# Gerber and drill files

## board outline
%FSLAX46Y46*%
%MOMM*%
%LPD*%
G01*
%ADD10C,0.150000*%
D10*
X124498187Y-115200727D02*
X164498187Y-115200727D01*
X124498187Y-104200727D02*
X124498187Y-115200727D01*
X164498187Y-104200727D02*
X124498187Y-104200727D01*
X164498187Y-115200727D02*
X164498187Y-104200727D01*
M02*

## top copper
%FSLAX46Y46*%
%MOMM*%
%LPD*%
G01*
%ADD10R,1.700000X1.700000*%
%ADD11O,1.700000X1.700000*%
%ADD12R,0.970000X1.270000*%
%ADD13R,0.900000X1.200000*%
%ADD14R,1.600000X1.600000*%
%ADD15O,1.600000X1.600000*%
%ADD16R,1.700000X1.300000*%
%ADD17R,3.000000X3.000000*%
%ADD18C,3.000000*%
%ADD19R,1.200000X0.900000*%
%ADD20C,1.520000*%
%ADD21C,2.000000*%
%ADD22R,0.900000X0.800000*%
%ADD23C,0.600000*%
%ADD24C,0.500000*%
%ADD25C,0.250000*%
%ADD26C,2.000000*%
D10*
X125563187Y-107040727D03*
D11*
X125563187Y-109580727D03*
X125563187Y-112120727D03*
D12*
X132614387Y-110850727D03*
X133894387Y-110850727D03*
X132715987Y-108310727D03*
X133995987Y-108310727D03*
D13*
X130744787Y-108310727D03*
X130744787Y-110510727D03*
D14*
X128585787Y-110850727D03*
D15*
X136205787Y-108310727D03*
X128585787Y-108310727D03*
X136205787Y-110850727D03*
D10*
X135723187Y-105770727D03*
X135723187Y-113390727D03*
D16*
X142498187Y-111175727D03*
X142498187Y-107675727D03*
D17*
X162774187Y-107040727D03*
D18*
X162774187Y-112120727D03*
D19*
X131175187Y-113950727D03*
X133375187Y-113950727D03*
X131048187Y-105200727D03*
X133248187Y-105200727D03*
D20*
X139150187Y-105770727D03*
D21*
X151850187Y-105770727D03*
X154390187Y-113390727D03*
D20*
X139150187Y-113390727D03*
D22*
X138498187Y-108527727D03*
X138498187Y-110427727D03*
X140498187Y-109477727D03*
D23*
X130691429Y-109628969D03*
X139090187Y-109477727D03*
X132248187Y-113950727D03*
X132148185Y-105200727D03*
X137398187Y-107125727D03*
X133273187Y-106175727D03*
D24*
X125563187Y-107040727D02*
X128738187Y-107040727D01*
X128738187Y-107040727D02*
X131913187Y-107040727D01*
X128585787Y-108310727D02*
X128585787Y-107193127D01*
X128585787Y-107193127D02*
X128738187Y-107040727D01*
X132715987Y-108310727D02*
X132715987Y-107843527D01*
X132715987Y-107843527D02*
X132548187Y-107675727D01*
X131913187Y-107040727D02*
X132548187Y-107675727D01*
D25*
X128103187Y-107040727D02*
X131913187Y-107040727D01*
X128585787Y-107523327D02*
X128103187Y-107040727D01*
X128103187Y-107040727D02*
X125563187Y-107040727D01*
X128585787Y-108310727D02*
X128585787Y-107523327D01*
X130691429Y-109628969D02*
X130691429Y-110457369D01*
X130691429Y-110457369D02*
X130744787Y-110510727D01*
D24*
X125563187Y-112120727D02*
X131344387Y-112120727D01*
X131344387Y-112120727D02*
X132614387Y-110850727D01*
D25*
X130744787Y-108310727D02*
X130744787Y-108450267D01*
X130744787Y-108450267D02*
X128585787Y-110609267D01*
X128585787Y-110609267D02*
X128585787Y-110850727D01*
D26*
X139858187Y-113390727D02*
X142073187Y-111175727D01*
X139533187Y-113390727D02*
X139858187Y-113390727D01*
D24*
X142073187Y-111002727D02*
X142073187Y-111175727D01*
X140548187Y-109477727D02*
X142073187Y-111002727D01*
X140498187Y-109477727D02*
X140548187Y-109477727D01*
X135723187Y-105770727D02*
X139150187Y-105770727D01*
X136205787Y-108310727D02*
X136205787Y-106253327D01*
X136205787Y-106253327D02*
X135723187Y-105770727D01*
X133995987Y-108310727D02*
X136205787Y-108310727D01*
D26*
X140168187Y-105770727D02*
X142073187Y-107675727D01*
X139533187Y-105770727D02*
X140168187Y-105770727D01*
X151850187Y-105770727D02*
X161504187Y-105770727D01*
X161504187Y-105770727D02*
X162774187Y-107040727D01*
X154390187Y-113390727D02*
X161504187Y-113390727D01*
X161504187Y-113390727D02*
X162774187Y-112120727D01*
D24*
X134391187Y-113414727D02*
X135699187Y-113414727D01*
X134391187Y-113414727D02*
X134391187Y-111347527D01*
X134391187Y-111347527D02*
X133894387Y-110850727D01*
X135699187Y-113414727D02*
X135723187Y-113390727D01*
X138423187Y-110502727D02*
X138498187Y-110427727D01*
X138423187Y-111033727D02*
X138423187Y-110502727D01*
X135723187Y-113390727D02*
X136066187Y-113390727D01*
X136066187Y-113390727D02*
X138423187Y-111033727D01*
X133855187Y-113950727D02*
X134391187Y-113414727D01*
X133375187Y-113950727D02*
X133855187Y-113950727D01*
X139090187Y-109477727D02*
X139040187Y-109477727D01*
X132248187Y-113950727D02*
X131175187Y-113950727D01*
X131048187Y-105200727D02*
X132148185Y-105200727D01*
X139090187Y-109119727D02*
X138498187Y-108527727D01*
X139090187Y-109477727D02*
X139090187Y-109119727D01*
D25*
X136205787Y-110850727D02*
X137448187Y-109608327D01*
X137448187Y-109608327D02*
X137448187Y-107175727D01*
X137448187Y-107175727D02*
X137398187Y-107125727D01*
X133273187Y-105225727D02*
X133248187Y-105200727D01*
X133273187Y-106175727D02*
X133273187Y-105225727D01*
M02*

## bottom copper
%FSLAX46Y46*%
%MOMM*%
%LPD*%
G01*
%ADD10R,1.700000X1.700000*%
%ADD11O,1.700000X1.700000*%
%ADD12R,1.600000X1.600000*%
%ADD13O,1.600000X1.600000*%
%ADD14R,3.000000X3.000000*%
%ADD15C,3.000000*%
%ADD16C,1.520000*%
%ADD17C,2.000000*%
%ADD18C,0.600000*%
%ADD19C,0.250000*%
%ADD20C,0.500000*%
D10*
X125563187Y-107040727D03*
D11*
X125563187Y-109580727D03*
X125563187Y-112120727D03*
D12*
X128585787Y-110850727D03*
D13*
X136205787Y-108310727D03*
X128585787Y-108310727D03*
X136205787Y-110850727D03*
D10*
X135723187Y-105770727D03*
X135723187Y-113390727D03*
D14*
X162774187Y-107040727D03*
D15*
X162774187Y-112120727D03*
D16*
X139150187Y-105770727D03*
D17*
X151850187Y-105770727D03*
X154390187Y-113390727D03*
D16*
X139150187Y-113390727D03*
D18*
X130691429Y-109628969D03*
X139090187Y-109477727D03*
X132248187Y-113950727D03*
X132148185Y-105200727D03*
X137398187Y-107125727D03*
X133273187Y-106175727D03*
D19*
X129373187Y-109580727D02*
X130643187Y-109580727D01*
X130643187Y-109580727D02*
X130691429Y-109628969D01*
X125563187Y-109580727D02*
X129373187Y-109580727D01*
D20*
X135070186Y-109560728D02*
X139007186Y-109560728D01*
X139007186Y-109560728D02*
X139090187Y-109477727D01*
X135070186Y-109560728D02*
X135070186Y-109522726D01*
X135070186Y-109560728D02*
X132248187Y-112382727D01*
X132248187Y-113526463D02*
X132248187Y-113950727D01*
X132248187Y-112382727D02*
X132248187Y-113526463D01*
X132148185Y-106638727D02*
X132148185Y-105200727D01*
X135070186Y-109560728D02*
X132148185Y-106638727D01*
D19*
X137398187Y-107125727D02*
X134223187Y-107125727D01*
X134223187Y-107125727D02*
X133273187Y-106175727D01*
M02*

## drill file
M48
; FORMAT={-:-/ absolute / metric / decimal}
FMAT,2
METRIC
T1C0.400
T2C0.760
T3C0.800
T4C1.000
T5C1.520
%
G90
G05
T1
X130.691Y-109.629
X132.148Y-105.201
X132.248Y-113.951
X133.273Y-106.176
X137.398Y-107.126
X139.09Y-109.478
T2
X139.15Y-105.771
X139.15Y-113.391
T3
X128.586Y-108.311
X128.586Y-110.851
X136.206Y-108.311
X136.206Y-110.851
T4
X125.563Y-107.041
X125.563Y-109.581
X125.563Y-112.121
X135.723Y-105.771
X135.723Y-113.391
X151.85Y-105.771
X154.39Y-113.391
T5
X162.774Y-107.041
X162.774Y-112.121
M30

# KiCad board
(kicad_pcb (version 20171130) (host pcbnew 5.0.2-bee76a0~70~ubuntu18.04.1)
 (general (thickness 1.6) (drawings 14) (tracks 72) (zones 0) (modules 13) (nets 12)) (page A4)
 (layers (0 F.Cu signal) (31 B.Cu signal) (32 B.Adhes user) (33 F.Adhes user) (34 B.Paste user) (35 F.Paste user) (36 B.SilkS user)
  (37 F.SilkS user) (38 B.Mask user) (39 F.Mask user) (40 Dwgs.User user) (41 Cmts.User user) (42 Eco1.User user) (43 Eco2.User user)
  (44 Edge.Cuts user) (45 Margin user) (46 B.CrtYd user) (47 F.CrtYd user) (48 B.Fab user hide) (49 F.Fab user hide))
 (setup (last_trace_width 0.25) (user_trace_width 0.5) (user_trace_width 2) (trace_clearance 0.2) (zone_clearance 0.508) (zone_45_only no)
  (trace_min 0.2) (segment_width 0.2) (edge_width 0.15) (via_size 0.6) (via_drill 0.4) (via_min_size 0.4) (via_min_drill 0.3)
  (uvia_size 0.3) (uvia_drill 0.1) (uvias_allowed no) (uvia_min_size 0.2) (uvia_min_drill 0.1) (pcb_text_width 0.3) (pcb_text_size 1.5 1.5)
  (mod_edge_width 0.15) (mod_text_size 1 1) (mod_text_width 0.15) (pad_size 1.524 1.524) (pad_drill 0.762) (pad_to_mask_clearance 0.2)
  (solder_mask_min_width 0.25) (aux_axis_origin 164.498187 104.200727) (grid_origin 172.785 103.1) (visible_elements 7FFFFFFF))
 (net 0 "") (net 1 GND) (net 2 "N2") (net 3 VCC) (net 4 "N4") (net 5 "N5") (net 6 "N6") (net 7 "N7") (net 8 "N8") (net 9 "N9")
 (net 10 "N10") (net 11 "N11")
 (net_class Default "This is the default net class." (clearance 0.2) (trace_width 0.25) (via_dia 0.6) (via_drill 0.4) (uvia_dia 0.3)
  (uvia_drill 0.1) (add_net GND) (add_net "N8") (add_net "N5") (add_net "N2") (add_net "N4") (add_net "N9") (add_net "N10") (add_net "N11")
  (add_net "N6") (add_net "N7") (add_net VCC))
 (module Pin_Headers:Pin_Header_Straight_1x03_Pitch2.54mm (layer B.Cu) (at 125.563187 107.040727 180)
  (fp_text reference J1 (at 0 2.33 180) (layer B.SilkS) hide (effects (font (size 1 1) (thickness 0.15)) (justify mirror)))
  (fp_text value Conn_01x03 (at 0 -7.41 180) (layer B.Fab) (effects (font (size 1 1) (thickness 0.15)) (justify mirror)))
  (pad 1 thru_hole rect (at 0 0 180) (size 1.7 1.7) (drill 1) (layers *.Cu *.Mask) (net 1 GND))
  (pad 2 thru_hole oval (at 0 -2.54 180) (size 1.7 1.7) (drill 1) (layers *.Cu *.Mask) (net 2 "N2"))
  (pad 3 thru_hole oval (at 0 -5.08 180) (size 1.7 1.7) (drill 1) (layers *.Cu *.Mask) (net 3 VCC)))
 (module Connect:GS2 (layer F.Cu) (at 133.254387 110.850727 90)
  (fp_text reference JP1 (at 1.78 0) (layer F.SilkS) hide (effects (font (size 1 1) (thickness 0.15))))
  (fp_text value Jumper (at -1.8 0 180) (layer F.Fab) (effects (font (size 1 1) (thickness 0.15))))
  (pad 1 smd rect (at 0 -0.64 90) (size 1.27 0.97) (layers F.Cu F.Paste F.Mask) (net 3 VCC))
  (pad 2 smd rect (at 0 0.64 90) (size 1.27 0.97) (layers F.Cu F.Paste F.Mask) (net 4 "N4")))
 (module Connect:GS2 (layer F.Cu) (at 133.355987 108.310727 90)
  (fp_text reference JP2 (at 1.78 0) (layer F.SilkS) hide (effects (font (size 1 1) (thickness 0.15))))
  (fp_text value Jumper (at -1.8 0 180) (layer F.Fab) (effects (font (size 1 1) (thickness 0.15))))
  (pad 1 smd rect (at 0 -0.64 90) (size 1.27 0.97) (layers F.Cu F.Paste F.Mask) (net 1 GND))
  (pad 2 smd rect (at 0 0.64 90) (size 1.27 0.97) (layers F.Cu F.Paste F.Mask) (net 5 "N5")))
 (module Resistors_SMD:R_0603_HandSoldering (layer F.Cu) (at 130.744787 109.410727 270)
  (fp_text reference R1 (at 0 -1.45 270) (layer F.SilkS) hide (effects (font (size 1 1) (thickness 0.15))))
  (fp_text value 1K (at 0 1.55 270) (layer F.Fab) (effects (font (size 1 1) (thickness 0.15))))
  (pad 1 smd rect (at -1.1 0 270) (size 1.2 0.9) (layers F.Cu F.Paste F.Mask) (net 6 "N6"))
  (pad 2 smd rect (at 1.1 0 270) (size 1.2 0.9) (layers F.Cu F.Paste F.Mask) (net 2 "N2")))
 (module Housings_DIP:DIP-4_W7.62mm (layer B.Cu) (at 128.585787 110.850727)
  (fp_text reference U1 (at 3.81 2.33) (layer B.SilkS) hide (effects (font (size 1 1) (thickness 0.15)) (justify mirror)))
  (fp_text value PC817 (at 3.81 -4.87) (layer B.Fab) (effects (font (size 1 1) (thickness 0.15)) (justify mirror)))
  (pad 1 thru_hole rect (at 0 0) (size 1.6 1.6) (drill 0.8) (layers *.Cu *.Mask) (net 6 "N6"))
  (pad 3 thru_hole oval (at 7.62 -2.54) (size 1.6 1.6) (drill 0.8) (layers *.Cu *.Mask) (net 5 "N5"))
  (pad 2 thru_hole oval (at 0 -2.54) (size 1.6 1.6) (drill 0.8) (layers *.Cu *.Mask) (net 1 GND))
  (pad 4 thru_hole oval (at 7.62 0) (size 1.6 1.6) (drill 0.8) (layers *.Cu *.Mask) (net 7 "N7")))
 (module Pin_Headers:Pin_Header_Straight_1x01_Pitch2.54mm (layer B.Cu) (at 135.723187 105.770727 270)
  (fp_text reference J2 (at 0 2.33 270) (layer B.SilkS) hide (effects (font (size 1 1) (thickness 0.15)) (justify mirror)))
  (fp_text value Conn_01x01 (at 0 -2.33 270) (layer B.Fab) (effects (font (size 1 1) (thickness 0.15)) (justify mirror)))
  (pad 1 thru_hole rect (at 0 0 270) (size 1.7 1.7) (drill 1) (layers *.Cu *.Mask) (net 5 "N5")))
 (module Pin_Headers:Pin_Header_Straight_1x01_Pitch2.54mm (layer B.Cu) (at 135.723187 113.390727)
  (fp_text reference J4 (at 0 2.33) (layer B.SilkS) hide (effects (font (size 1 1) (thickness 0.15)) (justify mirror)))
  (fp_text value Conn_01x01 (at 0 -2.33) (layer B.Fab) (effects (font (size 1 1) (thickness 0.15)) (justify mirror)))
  (pad 1 thru_hole rect (at 0 0) (size 1.7 1.7) (drill 1) (layers *.Cu *.Mask) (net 4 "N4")))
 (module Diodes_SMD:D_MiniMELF (layer F.Cu) (at 142.498187 109.425727 90)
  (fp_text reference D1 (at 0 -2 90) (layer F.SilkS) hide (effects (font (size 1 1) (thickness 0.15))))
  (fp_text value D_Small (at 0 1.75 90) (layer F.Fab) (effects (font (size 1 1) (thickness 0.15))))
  (pad 1 smd rect (at -1.75 0 90) (size 1.3 1.7) (layers F.Cu F.Paste F.Mask) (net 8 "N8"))
  (pad 2 smd rect (at 1.75 0 90) (size 1.3 1.7) (layers F.Cu F.Paste F.Mask) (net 5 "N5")))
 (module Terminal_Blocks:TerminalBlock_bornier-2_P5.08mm (layer B.Cu) (at 162.774187 107.040727 270)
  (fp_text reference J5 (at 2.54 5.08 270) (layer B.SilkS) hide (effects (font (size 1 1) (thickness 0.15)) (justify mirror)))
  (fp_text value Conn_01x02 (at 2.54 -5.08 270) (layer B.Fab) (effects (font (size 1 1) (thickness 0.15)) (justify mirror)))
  (pad 1 thru_hole rect (at 0 0 270) (size 3 3) (drill 1.52) (layers *.Cu *.Mask) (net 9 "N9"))
  (pad 2 thru_hole circle (at 5.08 0 270) (size 3 3) (drill 1.52) (layers *.Cu *.Mask) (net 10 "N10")))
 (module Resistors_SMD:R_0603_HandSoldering (layer F.Cu) (at 132.275187 113.950727)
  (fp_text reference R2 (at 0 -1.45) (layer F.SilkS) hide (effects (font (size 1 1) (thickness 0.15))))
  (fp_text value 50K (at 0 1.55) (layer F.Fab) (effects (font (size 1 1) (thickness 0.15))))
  (pad 1 smd rect (at -1.1 0) (size 1.2 0.9) (layers F.Cu F.Paste F.Mask) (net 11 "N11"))
  (pad 2 smd rect (at 1.1 0) (size 1.2 0.9) (layers F.Cu F.Paste F.Mask) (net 4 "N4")))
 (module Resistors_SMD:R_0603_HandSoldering (layer F.Cu) (at 132.148187 105.200727)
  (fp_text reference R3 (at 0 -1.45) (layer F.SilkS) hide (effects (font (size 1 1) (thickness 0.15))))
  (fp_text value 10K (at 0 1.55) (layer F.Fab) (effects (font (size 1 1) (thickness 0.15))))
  (pad 1 smd rect (at -1.1 0) (size 1.2 0.9) (layers F.Cu F.Paste F.Mask) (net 11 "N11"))
  (pad 2 smd rect (at 1.1 0) (size 1.2 0.9) (layers F.Cu F.Paste F.Mask) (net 7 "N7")))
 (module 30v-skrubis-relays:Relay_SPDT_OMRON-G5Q (layer B.Cu) (at 139.150187 105.770727)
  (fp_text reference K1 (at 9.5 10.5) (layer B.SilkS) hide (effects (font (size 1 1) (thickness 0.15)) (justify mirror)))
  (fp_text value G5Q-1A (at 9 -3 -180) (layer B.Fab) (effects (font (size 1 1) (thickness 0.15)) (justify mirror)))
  (pad 1 thru_hole circle (at 0 0 180) (size 1.52 1.52) (drill 0.76) (layers *.Cu *.Mask) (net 5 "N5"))
  (pad 2 thru_hole circle (at 12.7 0 180) (size 2 2) (drill 1) (layers *.Cu *.Mask) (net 9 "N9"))
  (pad 3 thru_hole circle (at 15.24 7.62 180) (size 2 2) (drill 1) (layers *.Cu *.Mask) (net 10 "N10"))
  (pad 5 thru_hole circle (at 0 7.62 180) (size 1.52 1.52) (drill 0.76) (layers *.Cu *.Mask) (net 8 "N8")))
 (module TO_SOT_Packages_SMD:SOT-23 (layer F.Cu) (at 139.498187 109.477727)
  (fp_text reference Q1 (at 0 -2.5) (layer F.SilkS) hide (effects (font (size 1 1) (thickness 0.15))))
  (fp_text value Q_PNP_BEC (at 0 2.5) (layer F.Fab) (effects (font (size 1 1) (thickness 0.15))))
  (pad 1 smd rect (at -1 -0.95) (size 0.9 0.8) (layers F.Cu F.Paste F.Mask) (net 11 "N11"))
  (pad 2 smd rect (at -1 0.95) (size 0.9 0.8) (layers F.Cu F.Paste F.Mask) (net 4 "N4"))
  (pad 3 smd rect (at 1 0) (size 0.9 0.8) (layers F.Cu F.Paste F.Mask) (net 8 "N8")))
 (gr_line (start 124.498187 115.200727) (end 164.498187 115.200727) (layer Edge.Cuts) (width 0.15))
 (gr_line (start 124.498187 104.200727) (end 124.498187 115.200727) (layer Edge.Cuts) (width 0.15))
 (gr_line (start 164.498187 104.200727) (end 124.498187 104.200727) (layer Edge.Cuts) (width 0.15))
 (gr_line (start 164.498187 115.200727) (end 164.498187 104.200727) (layer Edge.Cuts) (width 0.15))
 (segment (start 125.563187 107.040727) (end 128.738187 107.040727) (width 0.5) (layer F.Cu) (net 1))
 (segment (start 128.738187 107.040727) (end 131.913187 107.040727) (width 0.5) (layer F.Cu) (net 1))
 (segment (start 128.585787 108.310727) (end 128.585787 107.193127) (width 0.5) (layer F.Cu) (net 1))
 (segment (start 128.585787 107.193127) (end 128.738187 107.040727) (width 0.5) (layer F.Cu) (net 1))
 (segment (start 132.715987 108.310727) (end 132.715987 107.843527) (width 0.5) (layer F.Cu) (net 1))
 (segment (start 132.715987 107.843527) (end 132.548187 107.675727) (width 0.5) (layer F.Cu) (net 1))
 (segment (start 131.913187 107.040727) (end 132.548187 107.675727) (width 0.5) (layer F.Cu) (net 1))
 (segment (start 128.103187 107.040727) (end 131.913187 107.040727) (width 0.25) (layer F.Cu) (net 1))
 (segment (start 128.585787 107.523327) (end 128.103187 107.040727) (width 0.25) (layer F.Cu) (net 1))
 (segment (start 128.103187 107.040727) (end 125.563187 107.040727) (width 0.25) (layer F.Cu) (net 1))
 (segment (start 128.585787 108.310727) (end 128.585787 107.523327) (width 0.25) (layer F.Cu) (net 1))
 (segment (start 130.691429 109.628969) (end 130.691429 110.457369) (width 0.25) (layer F.Cu) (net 2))
 (segment (start 130.691429 110.457369) (end 130.744787 110.510727) (width 0.25) (layer F.Cu) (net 2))
 (segment (start 129.373187 109.580727) (end 130.643187 109.580727) (width 0.25) (layer B.Cu) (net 2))
 (segment (start 130.643187 109.580727) (end 130.691429 109.628969) (width 0.25) (layer B.Cu) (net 2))
 (via (at 130.691429 109.628969) (size 0.6) (drill 0.4) (layers F.Cu B.Cu) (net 2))
 (segment (start 125.563187 109.580727) (end 129.373187 109.580727) (width 0.25) (layer B.Cu) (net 2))
 (segment (start 125.563187 112.120727) (end 131.344387 112.120727) (width 0.5) (layer F.Cu) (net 3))
 (segment (start 131.344387 112.120727) (end 132.614387 110.850727) (width 0.5) (layer F.Cu) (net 3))
 (segment (start 130.744787 108.310727) (end 130.744787 108.450267) (width 0.25) (layer F.Cu) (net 6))
 (segment (start 130.744787 108.450267) (end 128.585787 110.609267) (width 0.25) (layer F.Cu) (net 6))
 (segment (start 128.585787 110.609267) (end 128.585787 110.850727) (width 0.25) (layer F.Cu) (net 6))
 (segment (start 139.858187 113.390727) (end 142.073187 111.175727) (width 2) (layer F.Cu) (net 8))
 (segment (start 139.533187 113.390727) (end 139.858187 113.390727) (width 2) (layer F.Cu) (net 8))
 (segment (start 142.073187 111.002727) (end 142.073187 111.175727) (width 0.5) (layer F.Cu) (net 8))
 (segment (start 140.548187 109.477727) (end 142.073187 111.002727) (width 0.5) (layer F.Cu) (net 8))
 (segment (start 140.498187 109.477727) (end 140.548187 109.477727) (width 0.5) (layer F.Cu) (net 8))
 (segment (start 135.723187 105.770727) (end 139.150187 105.770727) (width 0.5) (layer F.Cu) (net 5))
 (segment (start 136.205787 108.310727) (end 136.205787 106.253327) (width 0.5) (layer F.Cu) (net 5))
 (segment (start 136.205787 106.253327) (end 135.723187 105.770727) (width 0.5) (layer F.Cu) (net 5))
 (segment (start 133.995987 108.310727) (end 136.205787 108.310727) (width 0.5) (layer F.Cu) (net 5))
 (segment (start 140.168187 105.770727) (end 142.073187 107.675727) (width 2) (layer F.Cu) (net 5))
 (segment (start 139.533187 105.770727) (end 140.168187 105.770727) (width 2) (layer F.Cu) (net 5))
 (segment (start 151.850187 105.770727) (end 161.504187 105.770727) (width 2) (layer F.Cu) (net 9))
 (segment (start 161.504187 105.770727) (end 162.774187 107.040727) (width 2) (layer F.Cu) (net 9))
 (segment (start 154.390187 113.390727) (end 161.504187 113.390727) (width 2) (layer F.Cu) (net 10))
 (segment (start 161.504187 113.390727) (end 162.774187 112.120727) (width 2) (layer F.Cu) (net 10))
 (segment (start 134.391187 113.414727) (end 135.699187 113.414727) (width 0.5) (layer F.Cu) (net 4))
 (segment (start 134.391187 113.414727) (end 134.391187 111.347527) (width 0.5) (layer F.Cu) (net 4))
 (segment (start 134.391187 111.347527) (end 133.894387 110.850727) (width 0.5) (layer F.Cu) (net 4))
 (segment (start 135.699187 113.414727) (end 135.723187 113.390727) (width 0.5) (layer F.Cu) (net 4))
 (segment (start 138.423187 110.502727) (end 138.498187 110.427727) (width 0.5) (layer F.Cu) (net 4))
 (segment (start 138.423187 111.033727) (end 138.423187 110.502727) (width 0.5) (layer F.Cu) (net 4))
 (segment (start 135.723187 113.390727) (end 136.066187 113.390727) (width 0.5) (layer F.Cu) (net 4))
 (segment (start 136.066187 113.390727) (end 138.423187 111.033727) (width 0.5) (layer F.Cu) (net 4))
 (segment (start 133.855187 113.950727) (end 134.391187 113.414727) (width 0.5) (layer F.Cu) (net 4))
 (segment (start 133.375187 113.950727) (end 133.855187 113.950727) (width 0.5) (layer F.Cu) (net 4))
 (segment (start 139.090187 109.477727) (end 139.040187 109.477727) (width 0.5) (layer F.Cu) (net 11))
 (segment (start 135.070186 109.560728) (end 139.007186 109.560728) (width 0.5) (layer B.Cu) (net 11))
 (segment (start 139.007186 109.560728) (end 139.090187 109.477727) (width 0.5) (layer B.Cu) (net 11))
 (via (at 139.090187 109.477727) (size 0.6) (drill 0.4) (layers F.Cu B.Cu) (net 11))
 (segment (start 135.070186 109.560728) (end 135.070186 109.522726) (width 0.5) (layer B.Cu) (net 11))
 (segment (start 135.070186 109.560728) (end 132.248187 112.382727) (width 0.5) (layer B.Cu) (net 11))
 (via (at 132.248187 113.950727) (size 0.6) (drill 0.4) (layers F.Cu B.Cu) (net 11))
 (segment (start 132.248187 113.526463) (end 132.248187 113.950727) (width 0.5) (layer B.Cu) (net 11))
 (segment (start 132.248187 112.382727) (end 132.248187 113.526463) (width 0.5) (layer B.Cu) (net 11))
 (segment (start 132.248187 113.950727) (end 131.175187 113.950727) (width 0.5) (layer F.Cu) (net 11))
 (via (at 132.148185 105.200727) (size 0.6) (drill 0.4) (layers F.Cu B.Cu) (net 11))
 (segment (start 131.048187 105.200727) (end 132.148185 105.200727) (width 0.5) (layer F.Cu) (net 11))
 (segment (start 132.148185 106.638727) (end 132.148185 105.200727) (width 0.5) (layer B.Cu) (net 11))
 (segment (start 135.070186 109.560728) (end 132.148185 106.638727) (width 0.5) (layer B.Cu) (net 11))
 (segment (start 139.090187 109.119727) (end 138.498187 108.527727) (width 0.5) (layer F.Cu) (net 11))
 (segment (start 139.090187 109.477727) (end 139.090187 109.119727) (width 0.5) (layer F.Cu) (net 11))
 (segment (start 136.205787 110.850727) (end 137.448187 109.608327) (width 0.25) (layer F.Cu) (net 7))
 (via (at 137.398187 107.125727) (size 0.6) (drill 0.4) (layers F.Cu B.Cu) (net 7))
 (segment (start 137.448187 109.608327) (end 137.448187 107.175727) (width 0.25) (layer F.Cu) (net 7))
 (segment (start 137.448187 107.175727) (end 137.398187 107.125727) (width 0.25) (layer F.Cu) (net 7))
 (via (at 133.273187 106.175727) (size 0.6) (drill 0.4) (layers F.Cu B.Cu) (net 7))
 (segment (start 137.398187 107.125727) (end 134.223187 107.125727) (width 0.25) (layer B.Cu) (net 7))
 (segment (start 134.223187 107.125727) (end 133.273187 106.175727) (width 0.25) (layer B.Cu) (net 7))
 (segment (start 133.273187 105.225727) (end 133.248187 105.200727) (width 0.25) (layer F.Cu) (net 7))
 (segment (start 133.273187 106.175727) (end 133.273187 105.225727) (width 0.25) (layer F.Cu) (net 7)))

